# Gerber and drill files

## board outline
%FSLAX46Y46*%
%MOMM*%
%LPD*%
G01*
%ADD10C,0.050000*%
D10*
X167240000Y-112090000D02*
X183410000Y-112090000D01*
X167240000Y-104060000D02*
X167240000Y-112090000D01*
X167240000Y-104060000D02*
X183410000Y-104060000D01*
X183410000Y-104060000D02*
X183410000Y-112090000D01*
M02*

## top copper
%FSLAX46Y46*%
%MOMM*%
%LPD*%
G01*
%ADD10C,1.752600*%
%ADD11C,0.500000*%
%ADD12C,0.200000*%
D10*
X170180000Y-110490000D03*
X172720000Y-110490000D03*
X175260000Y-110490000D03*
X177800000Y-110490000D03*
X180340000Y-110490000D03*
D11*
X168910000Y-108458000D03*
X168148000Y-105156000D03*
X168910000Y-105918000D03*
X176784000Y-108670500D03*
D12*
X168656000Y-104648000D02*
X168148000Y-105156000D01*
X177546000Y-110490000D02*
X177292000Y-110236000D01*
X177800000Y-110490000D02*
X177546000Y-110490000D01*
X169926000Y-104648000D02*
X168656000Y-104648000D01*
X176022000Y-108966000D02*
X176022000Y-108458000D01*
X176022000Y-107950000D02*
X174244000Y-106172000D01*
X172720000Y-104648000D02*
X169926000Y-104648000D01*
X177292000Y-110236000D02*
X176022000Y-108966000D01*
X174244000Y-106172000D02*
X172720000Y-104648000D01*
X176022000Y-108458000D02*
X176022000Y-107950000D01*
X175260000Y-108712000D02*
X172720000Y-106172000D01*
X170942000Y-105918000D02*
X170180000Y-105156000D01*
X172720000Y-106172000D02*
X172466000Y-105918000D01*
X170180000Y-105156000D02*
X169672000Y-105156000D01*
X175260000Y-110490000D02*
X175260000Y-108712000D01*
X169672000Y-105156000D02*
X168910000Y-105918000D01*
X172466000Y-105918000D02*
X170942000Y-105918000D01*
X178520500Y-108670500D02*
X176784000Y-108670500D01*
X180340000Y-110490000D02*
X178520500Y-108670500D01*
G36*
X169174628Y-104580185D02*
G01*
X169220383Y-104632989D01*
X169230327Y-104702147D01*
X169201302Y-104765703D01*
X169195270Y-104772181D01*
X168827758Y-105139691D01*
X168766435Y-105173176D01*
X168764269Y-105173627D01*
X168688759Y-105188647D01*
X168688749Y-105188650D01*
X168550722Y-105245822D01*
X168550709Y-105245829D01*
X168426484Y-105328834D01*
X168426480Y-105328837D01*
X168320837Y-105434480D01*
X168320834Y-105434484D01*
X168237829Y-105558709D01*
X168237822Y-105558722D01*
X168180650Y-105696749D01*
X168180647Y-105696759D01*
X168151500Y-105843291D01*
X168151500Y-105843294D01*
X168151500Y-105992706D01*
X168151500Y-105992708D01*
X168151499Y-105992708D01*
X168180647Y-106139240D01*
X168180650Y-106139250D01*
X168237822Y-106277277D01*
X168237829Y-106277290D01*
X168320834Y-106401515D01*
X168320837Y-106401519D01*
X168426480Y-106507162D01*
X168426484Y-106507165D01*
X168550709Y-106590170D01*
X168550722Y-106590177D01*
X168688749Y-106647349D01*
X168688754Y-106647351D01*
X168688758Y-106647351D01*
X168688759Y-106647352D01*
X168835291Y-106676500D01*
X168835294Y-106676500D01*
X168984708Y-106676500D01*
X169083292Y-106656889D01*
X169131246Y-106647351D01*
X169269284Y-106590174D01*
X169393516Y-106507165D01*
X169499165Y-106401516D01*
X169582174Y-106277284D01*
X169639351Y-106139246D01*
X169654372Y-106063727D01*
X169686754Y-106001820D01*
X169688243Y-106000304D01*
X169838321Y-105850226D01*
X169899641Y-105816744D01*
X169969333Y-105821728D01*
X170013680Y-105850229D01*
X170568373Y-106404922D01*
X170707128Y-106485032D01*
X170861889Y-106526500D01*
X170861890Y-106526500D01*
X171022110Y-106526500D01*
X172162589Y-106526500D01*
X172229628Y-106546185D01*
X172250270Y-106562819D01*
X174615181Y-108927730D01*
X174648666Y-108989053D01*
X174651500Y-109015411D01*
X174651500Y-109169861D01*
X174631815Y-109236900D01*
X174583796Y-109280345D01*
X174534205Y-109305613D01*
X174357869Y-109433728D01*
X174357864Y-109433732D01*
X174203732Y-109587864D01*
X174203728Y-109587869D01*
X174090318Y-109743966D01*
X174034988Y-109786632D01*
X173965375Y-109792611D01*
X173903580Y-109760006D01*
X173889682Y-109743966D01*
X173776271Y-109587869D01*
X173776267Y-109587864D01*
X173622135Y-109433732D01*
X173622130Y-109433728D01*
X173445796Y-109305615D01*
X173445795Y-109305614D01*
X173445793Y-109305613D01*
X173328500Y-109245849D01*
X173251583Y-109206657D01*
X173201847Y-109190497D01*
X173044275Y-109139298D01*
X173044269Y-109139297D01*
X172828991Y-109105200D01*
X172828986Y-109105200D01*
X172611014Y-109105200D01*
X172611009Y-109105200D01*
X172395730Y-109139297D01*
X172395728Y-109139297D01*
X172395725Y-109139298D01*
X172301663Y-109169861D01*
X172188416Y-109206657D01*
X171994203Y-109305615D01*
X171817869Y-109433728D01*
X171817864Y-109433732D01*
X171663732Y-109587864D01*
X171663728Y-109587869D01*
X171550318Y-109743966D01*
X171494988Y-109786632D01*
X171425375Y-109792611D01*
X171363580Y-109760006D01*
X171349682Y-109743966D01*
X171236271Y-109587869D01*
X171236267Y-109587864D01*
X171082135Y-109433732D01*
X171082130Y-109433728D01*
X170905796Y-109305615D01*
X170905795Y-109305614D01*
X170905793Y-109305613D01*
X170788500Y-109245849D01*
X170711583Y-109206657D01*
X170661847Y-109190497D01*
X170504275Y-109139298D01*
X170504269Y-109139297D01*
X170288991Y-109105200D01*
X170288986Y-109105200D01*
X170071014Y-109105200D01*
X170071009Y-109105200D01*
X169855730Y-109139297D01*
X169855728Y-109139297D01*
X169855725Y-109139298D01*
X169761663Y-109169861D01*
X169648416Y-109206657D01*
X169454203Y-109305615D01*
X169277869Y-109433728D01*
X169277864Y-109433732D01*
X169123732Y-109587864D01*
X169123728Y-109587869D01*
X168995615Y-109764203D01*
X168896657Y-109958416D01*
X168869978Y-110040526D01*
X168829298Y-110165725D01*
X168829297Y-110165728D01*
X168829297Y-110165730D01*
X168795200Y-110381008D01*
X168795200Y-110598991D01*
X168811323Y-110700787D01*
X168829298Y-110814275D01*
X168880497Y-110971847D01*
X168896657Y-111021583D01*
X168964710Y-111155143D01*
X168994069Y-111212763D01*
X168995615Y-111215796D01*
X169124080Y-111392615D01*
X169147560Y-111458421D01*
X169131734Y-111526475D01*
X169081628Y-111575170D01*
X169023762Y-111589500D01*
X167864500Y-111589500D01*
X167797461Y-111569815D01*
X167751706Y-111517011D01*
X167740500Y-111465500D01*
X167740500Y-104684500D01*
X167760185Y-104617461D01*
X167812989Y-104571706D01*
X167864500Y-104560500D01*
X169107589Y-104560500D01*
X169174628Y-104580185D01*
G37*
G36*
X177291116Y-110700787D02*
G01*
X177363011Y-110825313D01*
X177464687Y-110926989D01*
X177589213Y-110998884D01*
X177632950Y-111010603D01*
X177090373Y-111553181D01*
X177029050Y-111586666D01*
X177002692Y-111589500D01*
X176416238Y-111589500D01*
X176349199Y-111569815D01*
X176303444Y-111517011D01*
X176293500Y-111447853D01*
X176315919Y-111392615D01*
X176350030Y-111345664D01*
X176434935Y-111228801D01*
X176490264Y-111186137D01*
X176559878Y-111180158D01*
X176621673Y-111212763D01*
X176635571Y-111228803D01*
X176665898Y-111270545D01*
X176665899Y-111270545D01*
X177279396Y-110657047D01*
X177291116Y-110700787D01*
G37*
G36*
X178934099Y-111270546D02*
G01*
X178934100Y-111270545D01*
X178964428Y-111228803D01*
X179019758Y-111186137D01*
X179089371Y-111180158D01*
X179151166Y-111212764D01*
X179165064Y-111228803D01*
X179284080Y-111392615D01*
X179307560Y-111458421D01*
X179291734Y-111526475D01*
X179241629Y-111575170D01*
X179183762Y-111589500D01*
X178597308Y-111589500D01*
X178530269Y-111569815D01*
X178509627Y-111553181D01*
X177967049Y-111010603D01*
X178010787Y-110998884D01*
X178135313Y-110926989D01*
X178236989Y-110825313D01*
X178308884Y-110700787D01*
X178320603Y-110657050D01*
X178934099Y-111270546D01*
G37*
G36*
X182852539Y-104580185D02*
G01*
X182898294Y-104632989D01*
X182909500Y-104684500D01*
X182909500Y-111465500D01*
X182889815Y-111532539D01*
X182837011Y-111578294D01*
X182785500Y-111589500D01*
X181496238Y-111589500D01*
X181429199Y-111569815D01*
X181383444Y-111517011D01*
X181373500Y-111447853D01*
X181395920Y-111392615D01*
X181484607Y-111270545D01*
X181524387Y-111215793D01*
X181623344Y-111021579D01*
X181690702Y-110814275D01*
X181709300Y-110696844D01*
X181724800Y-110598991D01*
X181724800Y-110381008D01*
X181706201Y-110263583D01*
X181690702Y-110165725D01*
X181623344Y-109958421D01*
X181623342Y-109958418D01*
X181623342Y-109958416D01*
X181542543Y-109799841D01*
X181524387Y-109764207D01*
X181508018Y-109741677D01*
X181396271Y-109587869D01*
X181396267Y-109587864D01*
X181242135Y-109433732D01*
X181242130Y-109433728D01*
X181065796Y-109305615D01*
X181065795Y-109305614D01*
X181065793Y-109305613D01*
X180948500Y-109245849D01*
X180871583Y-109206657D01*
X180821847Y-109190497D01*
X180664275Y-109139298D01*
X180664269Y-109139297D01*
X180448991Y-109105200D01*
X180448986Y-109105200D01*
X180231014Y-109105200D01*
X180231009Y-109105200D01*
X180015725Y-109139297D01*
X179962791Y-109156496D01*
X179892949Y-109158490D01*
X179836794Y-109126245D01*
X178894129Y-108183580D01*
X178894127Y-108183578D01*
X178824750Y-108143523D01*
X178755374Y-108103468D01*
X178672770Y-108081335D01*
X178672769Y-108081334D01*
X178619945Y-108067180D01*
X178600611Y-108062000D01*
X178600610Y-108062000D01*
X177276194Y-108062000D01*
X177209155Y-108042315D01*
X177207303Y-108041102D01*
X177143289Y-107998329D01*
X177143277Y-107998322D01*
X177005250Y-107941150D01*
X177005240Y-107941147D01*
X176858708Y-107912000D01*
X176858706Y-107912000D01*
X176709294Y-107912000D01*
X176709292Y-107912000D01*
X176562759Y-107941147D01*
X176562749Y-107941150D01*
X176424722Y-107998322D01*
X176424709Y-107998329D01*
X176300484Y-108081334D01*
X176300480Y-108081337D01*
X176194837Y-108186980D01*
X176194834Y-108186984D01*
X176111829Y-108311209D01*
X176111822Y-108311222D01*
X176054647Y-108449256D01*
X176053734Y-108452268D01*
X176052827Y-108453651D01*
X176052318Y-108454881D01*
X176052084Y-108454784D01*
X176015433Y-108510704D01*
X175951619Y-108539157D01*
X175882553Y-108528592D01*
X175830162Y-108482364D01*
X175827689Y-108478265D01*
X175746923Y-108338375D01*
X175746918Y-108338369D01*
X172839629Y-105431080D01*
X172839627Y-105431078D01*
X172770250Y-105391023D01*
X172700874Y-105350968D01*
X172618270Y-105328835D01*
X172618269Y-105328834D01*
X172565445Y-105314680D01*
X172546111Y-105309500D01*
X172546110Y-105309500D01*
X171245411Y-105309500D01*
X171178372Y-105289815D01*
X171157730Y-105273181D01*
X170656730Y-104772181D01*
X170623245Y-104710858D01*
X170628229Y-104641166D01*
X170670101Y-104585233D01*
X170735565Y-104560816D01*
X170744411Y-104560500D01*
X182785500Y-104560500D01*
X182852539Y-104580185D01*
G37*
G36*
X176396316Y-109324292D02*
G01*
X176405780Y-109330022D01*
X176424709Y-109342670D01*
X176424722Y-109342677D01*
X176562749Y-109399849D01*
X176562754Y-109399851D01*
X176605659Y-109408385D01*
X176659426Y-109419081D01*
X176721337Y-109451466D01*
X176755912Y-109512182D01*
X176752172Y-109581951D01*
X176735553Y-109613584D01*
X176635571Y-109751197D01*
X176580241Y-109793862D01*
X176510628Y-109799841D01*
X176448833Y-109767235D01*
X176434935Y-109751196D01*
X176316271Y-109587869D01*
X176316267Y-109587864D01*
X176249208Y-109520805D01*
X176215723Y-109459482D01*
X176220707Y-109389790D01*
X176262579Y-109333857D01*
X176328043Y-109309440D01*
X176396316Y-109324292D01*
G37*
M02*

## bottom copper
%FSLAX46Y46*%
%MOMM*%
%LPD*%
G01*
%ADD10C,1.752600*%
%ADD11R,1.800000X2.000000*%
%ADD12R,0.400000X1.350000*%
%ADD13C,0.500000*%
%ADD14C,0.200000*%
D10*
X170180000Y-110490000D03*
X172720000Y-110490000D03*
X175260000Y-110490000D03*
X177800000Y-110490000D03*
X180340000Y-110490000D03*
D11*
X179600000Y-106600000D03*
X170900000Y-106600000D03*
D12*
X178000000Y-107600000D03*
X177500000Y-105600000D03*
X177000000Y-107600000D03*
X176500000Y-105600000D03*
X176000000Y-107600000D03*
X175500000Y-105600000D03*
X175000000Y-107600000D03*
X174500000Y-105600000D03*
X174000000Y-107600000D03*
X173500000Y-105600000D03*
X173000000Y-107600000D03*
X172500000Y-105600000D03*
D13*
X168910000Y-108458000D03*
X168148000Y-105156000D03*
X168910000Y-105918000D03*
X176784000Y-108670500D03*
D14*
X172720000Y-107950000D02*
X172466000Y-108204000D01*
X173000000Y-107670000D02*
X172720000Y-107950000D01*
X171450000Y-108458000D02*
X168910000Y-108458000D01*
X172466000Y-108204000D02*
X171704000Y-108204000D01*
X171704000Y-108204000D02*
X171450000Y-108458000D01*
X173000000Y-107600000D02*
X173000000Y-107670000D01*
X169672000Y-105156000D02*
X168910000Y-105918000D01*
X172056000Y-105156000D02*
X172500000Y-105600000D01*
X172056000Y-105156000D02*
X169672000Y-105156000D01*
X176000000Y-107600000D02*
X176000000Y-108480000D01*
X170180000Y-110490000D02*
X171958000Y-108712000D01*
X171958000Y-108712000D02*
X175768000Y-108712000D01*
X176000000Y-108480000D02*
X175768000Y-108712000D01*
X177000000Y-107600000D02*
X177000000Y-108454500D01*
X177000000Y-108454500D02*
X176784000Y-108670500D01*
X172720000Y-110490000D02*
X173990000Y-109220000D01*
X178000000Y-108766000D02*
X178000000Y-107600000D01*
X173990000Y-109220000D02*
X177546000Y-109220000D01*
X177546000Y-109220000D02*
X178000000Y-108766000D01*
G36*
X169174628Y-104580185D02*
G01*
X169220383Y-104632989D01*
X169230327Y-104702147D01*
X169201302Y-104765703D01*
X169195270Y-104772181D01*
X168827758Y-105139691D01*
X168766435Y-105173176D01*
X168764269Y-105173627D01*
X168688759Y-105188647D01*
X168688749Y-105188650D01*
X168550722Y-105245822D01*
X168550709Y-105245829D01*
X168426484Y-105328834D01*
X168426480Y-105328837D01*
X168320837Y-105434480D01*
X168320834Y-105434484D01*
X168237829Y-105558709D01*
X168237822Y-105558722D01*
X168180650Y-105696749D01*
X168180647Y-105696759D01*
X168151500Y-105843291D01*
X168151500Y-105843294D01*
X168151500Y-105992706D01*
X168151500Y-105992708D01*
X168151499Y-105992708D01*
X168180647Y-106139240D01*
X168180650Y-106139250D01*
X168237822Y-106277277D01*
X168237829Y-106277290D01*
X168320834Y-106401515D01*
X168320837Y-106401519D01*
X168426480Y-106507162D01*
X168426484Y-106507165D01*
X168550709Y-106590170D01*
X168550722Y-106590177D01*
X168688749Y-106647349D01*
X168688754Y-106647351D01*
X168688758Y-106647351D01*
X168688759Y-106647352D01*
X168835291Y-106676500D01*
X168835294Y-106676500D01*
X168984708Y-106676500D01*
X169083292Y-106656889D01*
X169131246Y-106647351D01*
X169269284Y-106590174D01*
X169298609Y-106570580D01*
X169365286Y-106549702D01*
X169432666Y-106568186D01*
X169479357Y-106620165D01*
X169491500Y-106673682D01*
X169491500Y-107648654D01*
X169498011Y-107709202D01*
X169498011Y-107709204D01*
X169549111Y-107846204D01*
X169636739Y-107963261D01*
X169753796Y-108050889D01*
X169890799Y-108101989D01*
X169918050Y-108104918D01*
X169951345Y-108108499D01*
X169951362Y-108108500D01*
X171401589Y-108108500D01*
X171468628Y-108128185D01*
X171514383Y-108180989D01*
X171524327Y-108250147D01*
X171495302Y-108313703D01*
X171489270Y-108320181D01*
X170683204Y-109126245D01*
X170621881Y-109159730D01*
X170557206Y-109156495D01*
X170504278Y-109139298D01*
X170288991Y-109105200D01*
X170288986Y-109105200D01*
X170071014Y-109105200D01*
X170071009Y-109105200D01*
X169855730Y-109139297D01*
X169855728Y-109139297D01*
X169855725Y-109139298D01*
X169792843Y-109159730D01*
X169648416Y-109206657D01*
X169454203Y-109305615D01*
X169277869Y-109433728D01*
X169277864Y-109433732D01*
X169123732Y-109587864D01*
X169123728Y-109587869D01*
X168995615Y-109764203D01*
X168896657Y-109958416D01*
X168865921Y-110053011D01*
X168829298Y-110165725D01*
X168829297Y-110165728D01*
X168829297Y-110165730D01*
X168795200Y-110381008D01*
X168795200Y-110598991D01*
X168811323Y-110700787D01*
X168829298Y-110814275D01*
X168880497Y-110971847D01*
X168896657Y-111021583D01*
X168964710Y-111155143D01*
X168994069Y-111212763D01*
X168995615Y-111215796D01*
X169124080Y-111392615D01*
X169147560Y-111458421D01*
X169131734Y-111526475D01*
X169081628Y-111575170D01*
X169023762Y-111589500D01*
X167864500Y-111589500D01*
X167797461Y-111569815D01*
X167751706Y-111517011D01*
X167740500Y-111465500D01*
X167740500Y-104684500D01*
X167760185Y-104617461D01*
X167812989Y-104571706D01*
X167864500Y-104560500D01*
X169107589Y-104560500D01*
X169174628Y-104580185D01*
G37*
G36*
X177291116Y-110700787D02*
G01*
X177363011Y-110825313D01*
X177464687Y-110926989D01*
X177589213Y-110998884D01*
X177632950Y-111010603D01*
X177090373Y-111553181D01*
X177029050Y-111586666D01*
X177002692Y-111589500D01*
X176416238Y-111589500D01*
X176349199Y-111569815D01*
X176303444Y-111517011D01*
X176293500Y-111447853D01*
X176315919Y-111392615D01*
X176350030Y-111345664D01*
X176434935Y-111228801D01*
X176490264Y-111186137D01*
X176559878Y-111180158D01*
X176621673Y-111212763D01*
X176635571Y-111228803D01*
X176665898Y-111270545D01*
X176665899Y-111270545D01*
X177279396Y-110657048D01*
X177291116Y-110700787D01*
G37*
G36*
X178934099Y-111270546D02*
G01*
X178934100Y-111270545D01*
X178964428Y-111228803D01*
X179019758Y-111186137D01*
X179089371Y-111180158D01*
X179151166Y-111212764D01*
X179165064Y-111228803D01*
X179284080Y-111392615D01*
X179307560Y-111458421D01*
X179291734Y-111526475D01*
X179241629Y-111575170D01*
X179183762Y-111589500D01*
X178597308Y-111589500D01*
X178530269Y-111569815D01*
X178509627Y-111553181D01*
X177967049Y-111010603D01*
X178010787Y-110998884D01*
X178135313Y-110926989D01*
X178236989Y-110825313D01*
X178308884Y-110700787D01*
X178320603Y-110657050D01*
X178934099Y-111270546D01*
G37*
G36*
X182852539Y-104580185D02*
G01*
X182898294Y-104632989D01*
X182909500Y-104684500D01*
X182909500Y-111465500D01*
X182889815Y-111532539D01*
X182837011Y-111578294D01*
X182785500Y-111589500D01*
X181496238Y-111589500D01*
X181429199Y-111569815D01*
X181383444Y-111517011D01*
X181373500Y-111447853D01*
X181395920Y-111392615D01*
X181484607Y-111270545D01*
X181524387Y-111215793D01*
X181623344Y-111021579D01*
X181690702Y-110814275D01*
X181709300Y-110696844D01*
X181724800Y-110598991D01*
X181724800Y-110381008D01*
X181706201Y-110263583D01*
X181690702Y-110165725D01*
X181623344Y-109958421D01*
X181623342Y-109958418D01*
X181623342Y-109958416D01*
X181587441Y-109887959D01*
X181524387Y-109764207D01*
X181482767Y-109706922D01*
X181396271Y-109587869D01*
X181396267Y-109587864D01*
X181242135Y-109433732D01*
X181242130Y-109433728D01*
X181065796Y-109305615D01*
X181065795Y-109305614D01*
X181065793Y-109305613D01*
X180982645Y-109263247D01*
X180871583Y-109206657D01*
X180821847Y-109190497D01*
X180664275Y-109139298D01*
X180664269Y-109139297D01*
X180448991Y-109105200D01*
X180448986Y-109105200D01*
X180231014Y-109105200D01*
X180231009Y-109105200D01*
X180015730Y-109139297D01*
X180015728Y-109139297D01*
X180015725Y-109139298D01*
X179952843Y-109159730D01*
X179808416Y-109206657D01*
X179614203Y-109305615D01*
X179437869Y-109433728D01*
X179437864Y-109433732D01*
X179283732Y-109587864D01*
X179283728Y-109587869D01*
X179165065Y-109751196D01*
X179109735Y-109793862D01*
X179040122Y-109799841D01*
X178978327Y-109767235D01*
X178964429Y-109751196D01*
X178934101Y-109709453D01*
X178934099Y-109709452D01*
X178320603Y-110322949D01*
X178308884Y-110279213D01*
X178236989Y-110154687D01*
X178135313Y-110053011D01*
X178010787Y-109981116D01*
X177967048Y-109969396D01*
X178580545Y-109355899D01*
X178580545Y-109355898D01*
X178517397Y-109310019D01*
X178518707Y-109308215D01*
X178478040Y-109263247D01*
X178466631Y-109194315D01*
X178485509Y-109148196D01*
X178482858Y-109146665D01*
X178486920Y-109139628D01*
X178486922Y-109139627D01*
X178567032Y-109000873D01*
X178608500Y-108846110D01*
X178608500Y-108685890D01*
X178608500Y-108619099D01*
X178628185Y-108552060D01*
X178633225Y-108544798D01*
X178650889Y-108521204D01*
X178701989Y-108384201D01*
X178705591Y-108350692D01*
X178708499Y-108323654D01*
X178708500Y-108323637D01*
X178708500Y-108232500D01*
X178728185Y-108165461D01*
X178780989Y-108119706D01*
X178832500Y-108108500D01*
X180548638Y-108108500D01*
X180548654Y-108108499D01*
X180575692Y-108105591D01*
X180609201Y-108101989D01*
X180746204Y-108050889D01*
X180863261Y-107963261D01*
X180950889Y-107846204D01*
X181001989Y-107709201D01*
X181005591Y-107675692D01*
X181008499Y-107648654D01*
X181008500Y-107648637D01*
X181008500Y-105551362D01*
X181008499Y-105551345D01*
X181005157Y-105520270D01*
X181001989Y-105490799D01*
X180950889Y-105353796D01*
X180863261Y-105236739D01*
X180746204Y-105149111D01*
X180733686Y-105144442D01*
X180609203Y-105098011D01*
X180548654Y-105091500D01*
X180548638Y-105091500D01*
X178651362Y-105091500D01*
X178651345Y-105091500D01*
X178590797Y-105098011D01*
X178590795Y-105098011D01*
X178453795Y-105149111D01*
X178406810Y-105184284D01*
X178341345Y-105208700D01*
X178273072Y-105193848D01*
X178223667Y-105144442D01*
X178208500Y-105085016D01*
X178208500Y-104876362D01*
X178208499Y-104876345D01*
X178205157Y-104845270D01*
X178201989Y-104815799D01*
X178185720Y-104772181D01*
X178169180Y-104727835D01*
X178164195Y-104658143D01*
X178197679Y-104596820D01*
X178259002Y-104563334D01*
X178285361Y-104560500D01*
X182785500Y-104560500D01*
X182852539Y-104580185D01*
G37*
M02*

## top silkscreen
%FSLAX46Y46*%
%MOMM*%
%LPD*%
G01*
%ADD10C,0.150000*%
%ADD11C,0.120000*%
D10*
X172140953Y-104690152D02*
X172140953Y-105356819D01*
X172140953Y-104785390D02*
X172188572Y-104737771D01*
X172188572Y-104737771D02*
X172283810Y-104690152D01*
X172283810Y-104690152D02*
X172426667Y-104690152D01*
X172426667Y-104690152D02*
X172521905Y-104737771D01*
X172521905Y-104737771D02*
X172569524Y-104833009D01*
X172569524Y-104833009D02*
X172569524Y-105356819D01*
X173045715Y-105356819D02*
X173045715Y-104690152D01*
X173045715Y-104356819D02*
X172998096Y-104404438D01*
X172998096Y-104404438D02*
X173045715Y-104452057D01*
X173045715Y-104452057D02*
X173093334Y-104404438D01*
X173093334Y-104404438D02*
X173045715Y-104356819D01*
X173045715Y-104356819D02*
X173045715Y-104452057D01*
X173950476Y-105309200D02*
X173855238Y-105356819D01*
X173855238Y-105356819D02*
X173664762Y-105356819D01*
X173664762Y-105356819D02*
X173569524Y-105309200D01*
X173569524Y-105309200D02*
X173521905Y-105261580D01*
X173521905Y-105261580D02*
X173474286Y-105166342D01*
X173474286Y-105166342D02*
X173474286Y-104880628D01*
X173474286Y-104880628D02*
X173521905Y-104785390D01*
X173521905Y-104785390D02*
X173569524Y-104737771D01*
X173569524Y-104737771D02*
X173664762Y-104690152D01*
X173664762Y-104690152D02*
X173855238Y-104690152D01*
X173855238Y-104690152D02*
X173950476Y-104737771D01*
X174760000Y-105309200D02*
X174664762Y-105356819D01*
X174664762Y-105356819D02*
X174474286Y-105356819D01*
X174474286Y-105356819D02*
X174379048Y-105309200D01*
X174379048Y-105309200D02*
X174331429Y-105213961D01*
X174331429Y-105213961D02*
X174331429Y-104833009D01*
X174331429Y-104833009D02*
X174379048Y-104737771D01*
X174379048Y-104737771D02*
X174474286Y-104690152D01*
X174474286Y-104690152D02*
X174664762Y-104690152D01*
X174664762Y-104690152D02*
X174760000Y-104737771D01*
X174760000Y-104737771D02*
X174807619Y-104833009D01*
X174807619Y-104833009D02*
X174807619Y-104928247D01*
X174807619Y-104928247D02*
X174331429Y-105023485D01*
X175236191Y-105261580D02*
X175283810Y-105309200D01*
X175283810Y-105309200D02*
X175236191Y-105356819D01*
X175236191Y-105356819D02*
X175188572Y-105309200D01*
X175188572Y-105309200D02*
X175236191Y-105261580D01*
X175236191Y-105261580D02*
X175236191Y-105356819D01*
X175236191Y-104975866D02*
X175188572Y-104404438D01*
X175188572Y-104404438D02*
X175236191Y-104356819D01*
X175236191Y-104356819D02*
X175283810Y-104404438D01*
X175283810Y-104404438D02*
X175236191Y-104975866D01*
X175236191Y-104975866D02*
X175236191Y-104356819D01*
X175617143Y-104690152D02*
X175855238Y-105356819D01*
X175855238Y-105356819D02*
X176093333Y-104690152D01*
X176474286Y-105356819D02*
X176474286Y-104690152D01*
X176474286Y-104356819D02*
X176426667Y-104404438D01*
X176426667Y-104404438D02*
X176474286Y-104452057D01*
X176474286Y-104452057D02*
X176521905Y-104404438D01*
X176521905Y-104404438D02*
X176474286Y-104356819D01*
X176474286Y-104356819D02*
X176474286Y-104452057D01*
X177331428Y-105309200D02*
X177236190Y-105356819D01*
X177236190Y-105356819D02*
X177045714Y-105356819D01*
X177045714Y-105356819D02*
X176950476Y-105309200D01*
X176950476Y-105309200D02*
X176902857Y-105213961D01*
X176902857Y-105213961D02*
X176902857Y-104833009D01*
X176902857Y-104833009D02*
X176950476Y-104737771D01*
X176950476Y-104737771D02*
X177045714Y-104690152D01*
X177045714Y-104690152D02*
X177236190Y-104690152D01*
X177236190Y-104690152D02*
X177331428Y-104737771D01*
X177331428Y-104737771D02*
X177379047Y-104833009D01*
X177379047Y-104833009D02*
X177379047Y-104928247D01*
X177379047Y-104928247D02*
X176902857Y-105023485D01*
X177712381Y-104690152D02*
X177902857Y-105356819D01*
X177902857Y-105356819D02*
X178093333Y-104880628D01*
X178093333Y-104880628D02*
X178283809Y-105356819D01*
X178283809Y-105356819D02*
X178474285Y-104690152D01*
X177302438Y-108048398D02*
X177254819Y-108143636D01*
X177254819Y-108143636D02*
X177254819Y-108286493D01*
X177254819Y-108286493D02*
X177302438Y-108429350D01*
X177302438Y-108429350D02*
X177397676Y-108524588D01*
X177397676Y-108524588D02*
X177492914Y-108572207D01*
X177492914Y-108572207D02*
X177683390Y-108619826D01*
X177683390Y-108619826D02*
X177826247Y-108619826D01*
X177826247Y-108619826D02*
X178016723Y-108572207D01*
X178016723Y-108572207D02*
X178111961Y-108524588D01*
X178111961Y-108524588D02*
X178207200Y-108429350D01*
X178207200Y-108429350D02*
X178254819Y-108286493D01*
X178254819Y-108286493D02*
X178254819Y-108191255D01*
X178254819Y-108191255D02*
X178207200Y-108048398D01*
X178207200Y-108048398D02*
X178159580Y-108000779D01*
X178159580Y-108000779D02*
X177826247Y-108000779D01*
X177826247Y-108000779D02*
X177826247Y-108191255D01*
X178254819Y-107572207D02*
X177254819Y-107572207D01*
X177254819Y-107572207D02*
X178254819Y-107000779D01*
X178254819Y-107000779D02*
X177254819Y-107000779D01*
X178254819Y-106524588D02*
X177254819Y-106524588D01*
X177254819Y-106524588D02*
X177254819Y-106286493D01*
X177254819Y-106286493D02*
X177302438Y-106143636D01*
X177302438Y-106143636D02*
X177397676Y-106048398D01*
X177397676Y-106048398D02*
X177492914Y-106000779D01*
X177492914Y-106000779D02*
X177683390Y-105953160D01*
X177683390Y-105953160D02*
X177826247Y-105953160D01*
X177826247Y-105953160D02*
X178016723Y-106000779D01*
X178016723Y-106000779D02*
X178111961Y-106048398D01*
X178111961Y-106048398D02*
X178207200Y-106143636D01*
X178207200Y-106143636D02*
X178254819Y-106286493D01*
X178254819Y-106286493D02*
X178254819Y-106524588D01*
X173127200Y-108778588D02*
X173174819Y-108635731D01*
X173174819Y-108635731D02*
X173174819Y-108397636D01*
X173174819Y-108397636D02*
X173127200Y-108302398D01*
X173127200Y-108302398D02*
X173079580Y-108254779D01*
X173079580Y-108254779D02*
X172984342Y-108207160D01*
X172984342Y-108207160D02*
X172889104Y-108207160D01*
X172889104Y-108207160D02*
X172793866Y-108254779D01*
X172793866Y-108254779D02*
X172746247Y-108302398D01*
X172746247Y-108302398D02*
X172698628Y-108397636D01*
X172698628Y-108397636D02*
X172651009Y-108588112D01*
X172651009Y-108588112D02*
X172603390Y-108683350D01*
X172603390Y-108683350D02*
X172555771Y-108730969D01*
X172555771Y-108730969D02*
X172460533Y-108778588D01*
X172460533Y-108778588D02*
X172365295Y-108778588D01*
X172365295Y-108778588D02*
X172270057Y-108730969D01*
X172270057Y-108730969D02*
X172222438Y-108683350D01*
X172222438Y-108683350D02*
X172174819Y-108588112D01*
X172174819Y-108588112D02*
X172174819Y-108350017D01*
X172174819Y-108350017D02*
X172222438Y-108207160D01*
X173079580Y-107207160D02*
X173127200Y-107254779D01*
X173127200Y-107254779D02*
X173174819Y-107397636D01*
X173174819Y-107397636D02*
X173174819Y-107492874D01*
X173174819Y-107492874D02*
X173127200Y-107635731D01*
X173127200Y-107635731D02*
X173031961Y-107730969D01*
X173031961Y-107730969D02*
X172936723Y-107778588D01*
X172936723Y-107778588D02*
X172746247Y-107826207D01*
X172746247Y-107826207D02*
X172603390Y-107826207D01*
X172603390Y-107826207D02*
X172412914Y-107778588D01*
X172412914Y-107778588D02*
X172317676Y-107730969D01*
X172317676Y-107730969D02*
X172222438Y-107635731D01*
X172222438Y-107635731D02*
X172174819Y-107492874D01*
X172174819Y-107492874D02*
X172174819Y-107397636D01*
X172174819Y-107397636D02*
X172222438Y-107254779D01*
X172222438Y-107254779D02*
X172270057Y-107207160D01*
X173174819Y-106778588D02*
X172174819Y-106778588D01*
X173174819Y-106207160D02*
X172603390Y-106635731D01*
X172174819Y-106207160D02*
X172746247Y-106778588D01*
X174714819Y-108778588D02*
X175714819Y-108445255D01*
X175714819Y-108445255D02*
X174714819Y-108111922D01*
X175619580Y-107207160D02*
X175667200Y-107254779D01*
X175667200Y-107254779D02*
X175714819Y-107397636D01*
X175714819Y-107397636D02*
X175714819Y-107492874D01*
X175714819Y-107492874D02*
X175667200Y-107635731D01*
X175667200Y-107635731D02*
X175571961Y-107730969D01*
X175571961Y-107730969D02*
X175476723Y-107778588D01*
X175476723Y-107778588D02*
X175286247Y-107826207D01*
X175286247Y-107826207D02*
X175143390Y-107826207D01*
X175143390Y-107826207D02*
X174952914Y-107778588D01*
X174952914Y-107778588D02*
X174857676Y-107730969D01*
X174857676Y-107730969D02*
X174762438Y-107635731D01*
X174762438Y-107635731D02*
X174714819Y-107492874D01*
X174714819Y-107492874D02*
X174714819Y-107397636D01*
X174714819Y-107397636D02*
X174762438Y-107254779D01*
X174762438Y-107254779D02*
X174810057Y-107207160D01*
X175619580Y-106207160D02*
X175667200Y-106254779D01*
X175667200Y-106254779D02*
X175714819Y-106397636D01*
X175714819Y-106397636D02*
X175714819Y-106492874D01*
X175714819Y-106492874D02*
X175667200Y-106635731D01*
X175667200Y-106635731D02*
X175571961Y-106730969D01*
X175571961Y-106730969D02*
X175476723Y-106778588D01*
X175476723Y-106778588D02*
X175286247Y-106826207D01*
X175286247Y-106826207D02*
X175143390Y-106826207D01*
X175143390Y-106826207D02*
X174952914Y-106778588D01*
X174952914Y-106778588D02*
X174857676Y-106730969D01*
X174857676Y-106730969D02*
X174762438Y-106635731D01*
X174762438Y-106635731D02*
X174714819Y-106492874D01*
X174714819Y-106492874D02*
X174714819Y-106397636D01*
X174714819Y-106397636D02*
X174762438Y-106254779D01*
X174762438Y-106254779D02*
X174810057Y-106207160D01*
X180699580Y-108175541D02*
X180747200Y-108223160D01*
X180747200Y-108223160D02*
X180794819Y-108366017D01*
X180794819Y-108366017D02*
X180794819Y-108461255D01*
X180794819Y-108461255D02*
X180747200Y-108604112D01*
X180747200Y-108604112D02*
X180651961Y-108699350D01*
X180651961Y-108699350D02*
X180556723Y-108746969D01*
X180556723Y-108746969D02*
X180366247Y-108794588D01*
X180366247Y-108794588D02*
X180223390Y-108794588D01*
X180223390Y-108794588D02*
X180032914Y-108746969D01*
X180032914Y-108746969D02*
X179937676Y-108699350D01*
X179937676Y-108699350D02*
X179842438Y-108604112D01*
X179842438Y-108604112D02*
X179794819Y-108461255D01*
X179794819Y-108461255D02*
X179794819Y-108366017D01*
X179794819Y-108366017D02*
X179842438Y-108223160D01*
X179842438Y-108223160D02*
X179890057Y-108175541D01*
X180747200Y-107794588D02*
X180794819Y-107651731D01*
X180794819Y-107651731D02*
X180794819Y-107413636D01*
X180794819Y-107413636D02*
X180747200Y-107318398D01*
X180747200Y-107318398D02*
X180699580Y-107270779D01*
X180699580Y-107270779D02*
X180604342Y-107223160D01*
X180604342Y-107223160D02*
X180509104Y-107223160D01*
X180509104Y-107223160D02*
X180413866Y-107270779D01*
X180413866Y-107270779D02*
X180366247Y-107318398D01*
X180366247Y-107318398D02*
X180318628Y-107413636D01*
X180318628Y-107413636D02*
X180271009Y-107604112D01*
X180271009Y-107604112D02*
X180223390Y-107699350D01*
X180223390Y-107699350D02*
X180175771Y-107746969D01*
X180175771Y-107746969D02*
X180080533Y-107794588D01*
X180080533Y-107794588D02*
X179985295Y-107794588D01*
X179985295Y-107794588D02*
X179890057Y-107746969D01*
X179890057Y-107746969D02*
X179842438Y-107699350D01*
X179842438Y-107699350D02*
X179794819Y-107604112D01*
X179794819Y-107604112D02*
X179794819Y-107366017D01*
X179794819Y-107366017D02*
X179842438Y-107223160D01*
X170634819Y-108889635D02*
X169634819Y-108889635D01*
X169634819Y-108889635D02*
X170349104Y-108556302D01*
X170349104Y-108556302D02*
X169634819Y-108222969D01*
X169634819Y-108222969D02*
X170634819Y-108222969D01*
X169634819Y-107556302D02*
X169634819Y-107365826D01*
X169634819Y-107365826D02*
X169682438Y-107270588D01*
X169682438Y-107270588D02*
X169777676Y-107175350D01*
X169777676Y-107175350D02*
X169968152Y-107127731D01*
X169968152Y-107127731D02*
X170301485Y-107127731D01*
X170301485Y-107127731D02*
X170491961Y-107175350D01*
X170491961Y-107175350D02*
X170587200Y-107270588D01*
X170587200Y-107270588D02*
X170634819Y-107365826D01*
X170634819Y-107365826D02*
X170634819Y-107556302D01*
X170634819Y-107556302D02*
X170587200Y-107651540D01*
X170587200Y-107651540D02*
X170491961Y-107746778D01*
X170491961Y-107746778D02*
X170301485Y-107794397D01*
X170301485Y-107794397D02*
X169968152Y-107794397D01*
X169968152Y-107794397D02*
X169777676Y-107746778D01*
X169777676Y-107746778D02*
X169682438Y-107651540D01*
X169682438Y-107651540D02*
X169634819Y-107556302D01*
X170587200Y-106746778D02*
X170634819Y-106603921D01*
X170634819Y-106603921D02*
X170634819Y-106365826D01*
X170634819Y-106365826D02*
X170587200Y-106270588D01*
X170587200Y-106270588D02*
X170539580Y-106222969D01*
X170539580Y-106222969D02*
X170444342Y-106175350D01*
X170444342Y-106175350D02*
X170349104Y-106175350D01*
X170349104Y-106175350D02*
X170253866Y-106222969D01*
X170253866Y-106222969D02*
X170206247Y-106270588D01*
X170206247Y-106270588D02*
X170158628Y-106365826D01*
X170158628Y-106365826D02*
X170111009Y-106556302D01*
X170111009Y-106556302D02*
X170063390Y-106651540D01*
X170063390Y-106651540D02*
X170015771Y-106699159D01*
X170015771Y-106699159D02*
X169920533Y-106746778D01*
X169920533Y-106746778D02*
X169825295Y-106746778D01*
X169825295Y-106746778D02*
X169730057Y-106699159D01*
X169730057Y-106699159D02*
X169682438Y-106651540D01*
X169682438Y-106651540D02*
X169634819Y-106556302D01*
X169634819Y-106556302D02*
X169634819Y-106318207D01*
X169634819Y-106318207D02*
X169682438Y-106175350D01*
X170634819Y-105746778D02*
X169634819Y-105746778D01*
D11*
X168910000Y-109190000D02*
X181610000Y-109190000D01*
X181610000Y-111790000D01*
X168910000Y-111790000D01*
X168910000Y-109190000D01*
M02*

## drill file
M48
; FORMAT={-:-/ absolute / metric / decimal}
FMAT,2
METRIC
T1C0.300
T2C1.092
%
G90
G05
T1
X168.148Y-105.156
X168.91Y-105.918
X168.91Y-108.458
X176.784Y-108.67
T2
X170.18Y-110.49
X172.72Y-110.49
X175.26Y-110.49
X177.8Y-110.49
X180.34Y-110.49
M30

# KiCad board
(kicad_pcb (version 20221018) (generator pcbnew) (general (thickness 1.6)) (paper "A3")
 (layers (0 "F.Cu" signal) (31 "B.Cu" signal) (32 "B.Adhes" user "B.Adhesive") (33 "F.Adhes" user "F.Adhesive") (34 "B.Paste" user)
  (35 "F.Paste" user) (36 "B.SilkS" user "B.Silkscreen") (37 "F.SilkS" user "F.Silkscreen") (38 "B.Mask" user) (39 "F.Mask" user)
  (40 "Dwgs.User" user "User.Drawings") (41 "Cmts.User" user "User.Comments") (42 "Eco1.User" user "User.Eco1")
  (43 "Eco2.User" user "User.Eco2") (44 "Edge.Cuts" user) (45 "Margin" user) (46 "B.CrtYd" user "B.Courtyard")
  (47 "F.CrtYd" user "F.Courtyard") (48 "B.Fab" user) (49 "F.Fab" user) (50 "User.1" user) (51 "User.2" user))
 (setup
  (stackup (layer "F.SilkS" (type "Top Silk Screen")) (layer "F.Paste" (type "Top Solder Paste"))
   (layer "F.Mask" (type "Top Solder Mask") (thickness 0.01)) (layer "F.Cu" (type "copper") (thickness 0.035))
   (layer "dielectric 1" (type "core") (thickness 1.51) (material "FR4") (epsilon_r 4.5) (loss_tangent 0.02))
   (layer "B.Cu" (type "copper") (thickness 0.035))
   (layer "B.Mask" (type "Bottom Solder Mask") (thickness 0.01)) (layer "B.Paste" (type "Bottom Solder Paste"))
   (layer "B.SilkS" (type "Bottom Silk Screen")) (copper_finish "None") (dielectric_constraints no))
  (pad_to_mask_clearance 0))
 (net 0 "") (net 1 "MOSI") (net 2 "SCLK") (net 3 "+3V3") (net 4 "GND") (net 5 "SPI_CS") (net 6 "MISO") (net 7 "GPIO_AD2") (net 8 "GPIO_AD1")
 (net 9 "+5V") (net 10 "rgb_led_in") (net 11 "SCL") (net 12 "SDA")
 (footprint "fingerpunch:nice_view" (layer "F.Cu") (at 175.26 94.01)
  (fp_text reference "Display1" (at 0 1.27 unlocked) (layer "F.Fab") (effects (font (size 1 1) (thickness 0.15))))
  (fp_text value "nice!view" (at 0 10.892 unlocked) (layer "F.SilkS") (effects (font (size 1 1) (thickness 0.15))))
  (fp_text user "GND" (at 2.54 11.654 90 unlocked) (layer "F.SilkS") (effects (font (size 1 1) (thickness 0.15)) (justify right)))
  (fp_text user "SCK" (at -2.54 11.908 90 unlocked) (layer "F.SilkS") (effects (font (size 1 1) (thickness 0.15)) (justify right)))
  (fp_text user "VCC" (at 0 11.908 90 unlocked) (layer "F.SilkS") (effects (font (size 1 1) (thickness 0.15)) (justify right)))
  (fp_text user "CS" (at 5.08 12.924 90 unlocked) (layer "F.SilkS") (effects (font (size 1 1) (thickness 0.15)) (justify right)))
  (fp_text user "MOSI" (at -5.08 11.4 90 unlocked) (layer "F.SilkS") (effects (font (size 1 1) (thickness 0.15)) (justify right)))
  (fp_rect (start -6.35 15.18) (end 6.35 17.78) (stroke (width 0.12) (type solid)) (fill none) (layer "F.SilkS"))
  (pad "1" thru_hole circle (at -5.08 16.48) (size 1.7526 1.7526) (drill 1.0922) (layers "*.Cu" "*.Mask") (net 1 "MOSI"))
  (pad "2" thru_hole circle (at -2.54 16.48) (size 1.7526 1.7526) (drill 1.0922) (layers "*.Cu" "*.Mask") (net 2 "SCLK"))
  (pad "3" thru_hole circle (at 0 16.48) (size 1.7526 1.7526) (drill 1.0922) (layers "*.Cu" "*.Mask") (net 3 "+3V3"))
  (pad "4" thru_hole circle (at 2.54 16.48) (size 1.7526 1.7526) (drill 1.0922) (layers "*.Cu" "*.Mask") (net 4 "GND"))
  (pad "5" thru_hole circle (at 5.08 16.48) (size 1.7526 1.7526) (drill 1.0922) (layers "*.Cu" "*.Mask") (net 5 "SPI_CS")))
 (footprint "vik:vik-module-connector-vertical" (layer "B.Cu") (at 175.25 106.6 180)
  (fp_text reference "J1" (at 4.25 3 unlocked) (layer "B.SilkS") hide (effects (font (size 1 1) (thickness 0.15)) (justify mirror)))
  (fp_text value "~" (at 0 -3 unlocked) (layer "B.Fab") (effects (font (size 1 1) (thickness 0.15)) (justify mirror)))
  (pad "" smd rect (at -4.35 0 180) (size 1.8 2) (layers "B.Cu" "B.Paste" "B.Mask") (thermal_bridge_angle 45))
  (pad "" smd rect (at 4.35 0 180) (size 1.8 2) (layers "B.Cu" "B.Paste" "B.Mask") (thermal_bridge_angle 45))
  (pad "1" smd rect (at -2.75 -1 180) (size 0.4 1.35) (layers "B.Cu" "B.Paste" "B.Mask") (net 2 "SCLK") (thermal_bridge_angle 45))
  (pad "2" smd rect (at -2.25 1 180) (size 0.4 1.35) (layers "B.Cu" "B.Paste" "B.Mask") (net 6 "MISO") (thermal_bridge_angle 45))
  (pad "3" smd rect (at -1.75 -1 180) (size 0.4 1.35) (layers "B.Cu" "B.Paste" "B.Mask") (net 5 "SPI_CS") (thermal_bridge_angle 45))
  (pad "4" smd rect (at -1.25 1 180) (size 0.4 1.35) (layers "B.Cu" "B.Paste" "B.Mask") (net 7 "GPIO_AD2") (thermal_bridge_angle 45))
  (pad "5" smd rect (at -0.75 -1 180) (size 0.4 1.35) (layers "B.Cu" "B.Paste" "B.Mask") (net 1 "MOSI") (thermal_bridge_angle 45))
  (pad "6" smd rect (at -0.25 1 180) (size 0.4 1.35) (layers "B.Cu" "B.Paste" "B.Mask") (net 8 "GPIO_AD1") (thermal_bridge_angle 45))
  (pad "7" smd rect (at 0.25 -1 180) (size 0.4 1.35) (layers "B.Cu" "B.Paste" "B.Mask") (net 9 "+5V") (thermal_bridge_angle 45))
  (pad "8" smd rect (at 0.75 1 180) (size 0.4 1.35) (layers "B.Cu" "B.Paste" "B.Mask") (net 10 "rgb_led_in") (thermal_bridge_angle 45))
  (pad "9" smd rect (at 1.25 -1 180) (size 0.4 1.35) (layers "B.Cu" "B.Paste" "B.Mask") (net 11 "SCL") (thermal_bridge_angle 45))
  (pad "10" smd rect (at 1.75 1 180) (size 0.4 1.35) (layers "B.Cu" "B.Paste" "B.Mask") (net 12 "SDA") (thermal_bridge_angle 45))
  (pad "11" smd rect (at 2.25 -1 180) (size 0.4 1.35) (layers "B.Cu" "B.Paste" "B.Mask") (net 4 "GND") (thermal_bridge_angle 45))
  (pad "12" smd rect (at 2.75 1 180) (size 0.4 1.35) (layers "B.Cu" "B.Paste" "B.Mask") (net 3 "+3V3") (thermal_bridge_angle 45)))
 (gr_line (start 167.24 112.09) (end 183.41 112.09) (stroke (width 0.05) (type default)) (layer "Edge.Cuts"))
 (gr_line (start 167.24 104.06) (end 167.24 112.09) (stroke (width 0.05) (type default)) (layer "Edge.Cuts"))
 (gr_line (start 167.24 104.06) (end 183.41 104.06) (stroke (width 0.05) (type default)) (layer "Edge.Cuts"))
 (gr_line (start 183.41 104.06) (end 183.41 112.09) (stroke (width 0.05) (type default)) (layer "Edge.Cuts"))
 (segment (start 168.656 104.648) (end 168.148 105.156) (width 0.2) (layer "F.Cu") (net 4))
 (segment (start 177.546 110.49) (end 177.292 110.236) (width 0.2) (layer "F.Cu") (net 4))
 (segment (start 177.8 110.49) (end 177.546 110.49) (width 0.2) (layer "F.Cu") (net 4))
 (segment (start 169.926 104.648) (end 168.656 104.648) (width 0.2) (layer "F.Cu") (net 4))
 (segment (start 176.022 108.966) (end 176.022 108.458) (width 0.2) (layer "F.Cu") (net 4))
 (segment (start 176.022 107.95) (end 174.244 106.172) (width 0.2) (layer "F.Cu") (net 4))
 (segment (start 172.72 104.648) (end 169.926 104.648) (width 0.2) (layer "F.Cu") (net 4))
 (segment (start 177.292 110.236) (end 176.022 108.966) (width 0.2) (layer "F.Cu") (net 4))
 (segment (start 174.244 106.172) (end 172.72 104.648) (width 0.2) (layer "F.Cu") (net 4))
 (segment (start 176.022 108.458) (end 176.022 107.95) (width 0.2) (layer "F.Cu") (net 4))
 (via (at 168.91 108.458) (size 0.5) (drill 0.3) (layers "F.Cu" "B.Cu") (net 4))
 (via (at 168.148 105.156) (size 0.5) (drill 0.3) (layers "F.Cu" "B.Cu") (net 4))
 (segment (start 172.72 107.95) (end 172.466 108.204) (width 0.2) (layer "B.Cu") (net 4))
 (segment (start 173 107.67) (end 172.72 107.95) (width 0.2) (layer "B.Cu") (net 4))
 (segment (start 171.45 108.458) (end 168.91 108.458) (width 0.2) (layer "B.Cu") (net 4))
 (segment (start 172.466 108.204) (end 171.704 108.204) (width 0.2) (layer "B.Cu") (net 4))
 (segment (start 171.704 108.204) (end 171.45 108.458) (width 0.2) (layer "B.Cu") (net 4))
 (segment (start 173 107.6) (end 173 107.67) (width 0.2) (layer "B.Cu") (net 4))
 (segment (start 175.26 108.712) (end 172.72 106.172) (width 0.2) (layer "F.Cu") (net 3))
 (segment (start 170.942 105.918) (end 170.18 105.156) (width 0.2) (layer "F.Cu") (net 3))
 (segment (start 172.72 106.172) (end 172.466 105.918) (width 0.2) (layer "F.Cu") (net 3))
 (segment (start 170.18 105.156) (end 169.672 105.156) (width 0.2) (layer "F.Cu") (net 3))
 (segment (start 175.26 110.49) (end 175.26 108.712) (width 0.2) (layer "F.Cu") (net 3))
 (segment (start 169.672 105.156) (end 168.91 105.918) (width 0.2) (layer "F.Cu") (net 3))
 (segment (start 172.466 105.918) (end 170.942 105.918) (width 0.2) (layer "F.Cu") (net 3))
 (via (at 168.91 105.918) (size 0.5) (drill 0.3) (layers "F.Cu" "B.Cu") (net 3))
 (segment (start 169.672 105.156) (end 168.91 105.918) (width 0.2) (layer "B.Cu") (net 3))
 (segment (start 172.056 105.156) (end 172.5 105.6) (width 0.2) (layer "B.Cu") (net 3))
 (segment (start 172.056 105.156) (end 169.672 105.156) (width 0.2) (layer "B.Cu") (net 3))
 (segment (start 176 107.6) (end 176 108.48) (width 0.2) (layer "B.Cu") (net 1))
 (segment (start 170.18 110.49) (end 171.958 108.712) (width 0.2) (layer "B.Cu") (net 1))
 (segment (start 171.958 108.712) (end 175.768 108.712) (width 0.2) (layer "B.Cu") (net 1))
 (segment (start 176 108.48) (end 175.768 108.712) (width 0.2) (layer "B.Cu") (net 1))
 (segment (start 178.5205 108.6705) (end 176.784 108.6705) (width 0.2) (layer "F.Cu") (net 5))
 (segment (start 180.34 110.49) (end 178.5205 108.6705) (width 0.2) (layer "F.Cu") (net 5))
 (via (at 176.784 108.6705) (size 0.5) (drill 0.3) (layers "F.Cu" "B.Cu") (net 5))
 (segment (start 177 107.6) (end 177 108.4545) (width 0.2) (layer "B.Cu") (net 5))
 (segment (start 177 108.4545) (end 176.784 108.6705) (width 0.2) (layer "B.Cu") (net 5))
 (segment (start 172.72 110.49) (end 173.99 109.22) (width 0.2) (layer "B.Cu") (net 2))
 (segment (start 178 108.766) (end 178 107.6) (width 0.2) (layer "B.Cu") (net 2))
 (segment (start 173.99 109.22) (end 177.546 109.22) (width 0.2) (layer "B.Cu") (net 2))
 (segment (start 177.546 109.22) (end 178 108.766) (width 0.2) (layer "B.Cu") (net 2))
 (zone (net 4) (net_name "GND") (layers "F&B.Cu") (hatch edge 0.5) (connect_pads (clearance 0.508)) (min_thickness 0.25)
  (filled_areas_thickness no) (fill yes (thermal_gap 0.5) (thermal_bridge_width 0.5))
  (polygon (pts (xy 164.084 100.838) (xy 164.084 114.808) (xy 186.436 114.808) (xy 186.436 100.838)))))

